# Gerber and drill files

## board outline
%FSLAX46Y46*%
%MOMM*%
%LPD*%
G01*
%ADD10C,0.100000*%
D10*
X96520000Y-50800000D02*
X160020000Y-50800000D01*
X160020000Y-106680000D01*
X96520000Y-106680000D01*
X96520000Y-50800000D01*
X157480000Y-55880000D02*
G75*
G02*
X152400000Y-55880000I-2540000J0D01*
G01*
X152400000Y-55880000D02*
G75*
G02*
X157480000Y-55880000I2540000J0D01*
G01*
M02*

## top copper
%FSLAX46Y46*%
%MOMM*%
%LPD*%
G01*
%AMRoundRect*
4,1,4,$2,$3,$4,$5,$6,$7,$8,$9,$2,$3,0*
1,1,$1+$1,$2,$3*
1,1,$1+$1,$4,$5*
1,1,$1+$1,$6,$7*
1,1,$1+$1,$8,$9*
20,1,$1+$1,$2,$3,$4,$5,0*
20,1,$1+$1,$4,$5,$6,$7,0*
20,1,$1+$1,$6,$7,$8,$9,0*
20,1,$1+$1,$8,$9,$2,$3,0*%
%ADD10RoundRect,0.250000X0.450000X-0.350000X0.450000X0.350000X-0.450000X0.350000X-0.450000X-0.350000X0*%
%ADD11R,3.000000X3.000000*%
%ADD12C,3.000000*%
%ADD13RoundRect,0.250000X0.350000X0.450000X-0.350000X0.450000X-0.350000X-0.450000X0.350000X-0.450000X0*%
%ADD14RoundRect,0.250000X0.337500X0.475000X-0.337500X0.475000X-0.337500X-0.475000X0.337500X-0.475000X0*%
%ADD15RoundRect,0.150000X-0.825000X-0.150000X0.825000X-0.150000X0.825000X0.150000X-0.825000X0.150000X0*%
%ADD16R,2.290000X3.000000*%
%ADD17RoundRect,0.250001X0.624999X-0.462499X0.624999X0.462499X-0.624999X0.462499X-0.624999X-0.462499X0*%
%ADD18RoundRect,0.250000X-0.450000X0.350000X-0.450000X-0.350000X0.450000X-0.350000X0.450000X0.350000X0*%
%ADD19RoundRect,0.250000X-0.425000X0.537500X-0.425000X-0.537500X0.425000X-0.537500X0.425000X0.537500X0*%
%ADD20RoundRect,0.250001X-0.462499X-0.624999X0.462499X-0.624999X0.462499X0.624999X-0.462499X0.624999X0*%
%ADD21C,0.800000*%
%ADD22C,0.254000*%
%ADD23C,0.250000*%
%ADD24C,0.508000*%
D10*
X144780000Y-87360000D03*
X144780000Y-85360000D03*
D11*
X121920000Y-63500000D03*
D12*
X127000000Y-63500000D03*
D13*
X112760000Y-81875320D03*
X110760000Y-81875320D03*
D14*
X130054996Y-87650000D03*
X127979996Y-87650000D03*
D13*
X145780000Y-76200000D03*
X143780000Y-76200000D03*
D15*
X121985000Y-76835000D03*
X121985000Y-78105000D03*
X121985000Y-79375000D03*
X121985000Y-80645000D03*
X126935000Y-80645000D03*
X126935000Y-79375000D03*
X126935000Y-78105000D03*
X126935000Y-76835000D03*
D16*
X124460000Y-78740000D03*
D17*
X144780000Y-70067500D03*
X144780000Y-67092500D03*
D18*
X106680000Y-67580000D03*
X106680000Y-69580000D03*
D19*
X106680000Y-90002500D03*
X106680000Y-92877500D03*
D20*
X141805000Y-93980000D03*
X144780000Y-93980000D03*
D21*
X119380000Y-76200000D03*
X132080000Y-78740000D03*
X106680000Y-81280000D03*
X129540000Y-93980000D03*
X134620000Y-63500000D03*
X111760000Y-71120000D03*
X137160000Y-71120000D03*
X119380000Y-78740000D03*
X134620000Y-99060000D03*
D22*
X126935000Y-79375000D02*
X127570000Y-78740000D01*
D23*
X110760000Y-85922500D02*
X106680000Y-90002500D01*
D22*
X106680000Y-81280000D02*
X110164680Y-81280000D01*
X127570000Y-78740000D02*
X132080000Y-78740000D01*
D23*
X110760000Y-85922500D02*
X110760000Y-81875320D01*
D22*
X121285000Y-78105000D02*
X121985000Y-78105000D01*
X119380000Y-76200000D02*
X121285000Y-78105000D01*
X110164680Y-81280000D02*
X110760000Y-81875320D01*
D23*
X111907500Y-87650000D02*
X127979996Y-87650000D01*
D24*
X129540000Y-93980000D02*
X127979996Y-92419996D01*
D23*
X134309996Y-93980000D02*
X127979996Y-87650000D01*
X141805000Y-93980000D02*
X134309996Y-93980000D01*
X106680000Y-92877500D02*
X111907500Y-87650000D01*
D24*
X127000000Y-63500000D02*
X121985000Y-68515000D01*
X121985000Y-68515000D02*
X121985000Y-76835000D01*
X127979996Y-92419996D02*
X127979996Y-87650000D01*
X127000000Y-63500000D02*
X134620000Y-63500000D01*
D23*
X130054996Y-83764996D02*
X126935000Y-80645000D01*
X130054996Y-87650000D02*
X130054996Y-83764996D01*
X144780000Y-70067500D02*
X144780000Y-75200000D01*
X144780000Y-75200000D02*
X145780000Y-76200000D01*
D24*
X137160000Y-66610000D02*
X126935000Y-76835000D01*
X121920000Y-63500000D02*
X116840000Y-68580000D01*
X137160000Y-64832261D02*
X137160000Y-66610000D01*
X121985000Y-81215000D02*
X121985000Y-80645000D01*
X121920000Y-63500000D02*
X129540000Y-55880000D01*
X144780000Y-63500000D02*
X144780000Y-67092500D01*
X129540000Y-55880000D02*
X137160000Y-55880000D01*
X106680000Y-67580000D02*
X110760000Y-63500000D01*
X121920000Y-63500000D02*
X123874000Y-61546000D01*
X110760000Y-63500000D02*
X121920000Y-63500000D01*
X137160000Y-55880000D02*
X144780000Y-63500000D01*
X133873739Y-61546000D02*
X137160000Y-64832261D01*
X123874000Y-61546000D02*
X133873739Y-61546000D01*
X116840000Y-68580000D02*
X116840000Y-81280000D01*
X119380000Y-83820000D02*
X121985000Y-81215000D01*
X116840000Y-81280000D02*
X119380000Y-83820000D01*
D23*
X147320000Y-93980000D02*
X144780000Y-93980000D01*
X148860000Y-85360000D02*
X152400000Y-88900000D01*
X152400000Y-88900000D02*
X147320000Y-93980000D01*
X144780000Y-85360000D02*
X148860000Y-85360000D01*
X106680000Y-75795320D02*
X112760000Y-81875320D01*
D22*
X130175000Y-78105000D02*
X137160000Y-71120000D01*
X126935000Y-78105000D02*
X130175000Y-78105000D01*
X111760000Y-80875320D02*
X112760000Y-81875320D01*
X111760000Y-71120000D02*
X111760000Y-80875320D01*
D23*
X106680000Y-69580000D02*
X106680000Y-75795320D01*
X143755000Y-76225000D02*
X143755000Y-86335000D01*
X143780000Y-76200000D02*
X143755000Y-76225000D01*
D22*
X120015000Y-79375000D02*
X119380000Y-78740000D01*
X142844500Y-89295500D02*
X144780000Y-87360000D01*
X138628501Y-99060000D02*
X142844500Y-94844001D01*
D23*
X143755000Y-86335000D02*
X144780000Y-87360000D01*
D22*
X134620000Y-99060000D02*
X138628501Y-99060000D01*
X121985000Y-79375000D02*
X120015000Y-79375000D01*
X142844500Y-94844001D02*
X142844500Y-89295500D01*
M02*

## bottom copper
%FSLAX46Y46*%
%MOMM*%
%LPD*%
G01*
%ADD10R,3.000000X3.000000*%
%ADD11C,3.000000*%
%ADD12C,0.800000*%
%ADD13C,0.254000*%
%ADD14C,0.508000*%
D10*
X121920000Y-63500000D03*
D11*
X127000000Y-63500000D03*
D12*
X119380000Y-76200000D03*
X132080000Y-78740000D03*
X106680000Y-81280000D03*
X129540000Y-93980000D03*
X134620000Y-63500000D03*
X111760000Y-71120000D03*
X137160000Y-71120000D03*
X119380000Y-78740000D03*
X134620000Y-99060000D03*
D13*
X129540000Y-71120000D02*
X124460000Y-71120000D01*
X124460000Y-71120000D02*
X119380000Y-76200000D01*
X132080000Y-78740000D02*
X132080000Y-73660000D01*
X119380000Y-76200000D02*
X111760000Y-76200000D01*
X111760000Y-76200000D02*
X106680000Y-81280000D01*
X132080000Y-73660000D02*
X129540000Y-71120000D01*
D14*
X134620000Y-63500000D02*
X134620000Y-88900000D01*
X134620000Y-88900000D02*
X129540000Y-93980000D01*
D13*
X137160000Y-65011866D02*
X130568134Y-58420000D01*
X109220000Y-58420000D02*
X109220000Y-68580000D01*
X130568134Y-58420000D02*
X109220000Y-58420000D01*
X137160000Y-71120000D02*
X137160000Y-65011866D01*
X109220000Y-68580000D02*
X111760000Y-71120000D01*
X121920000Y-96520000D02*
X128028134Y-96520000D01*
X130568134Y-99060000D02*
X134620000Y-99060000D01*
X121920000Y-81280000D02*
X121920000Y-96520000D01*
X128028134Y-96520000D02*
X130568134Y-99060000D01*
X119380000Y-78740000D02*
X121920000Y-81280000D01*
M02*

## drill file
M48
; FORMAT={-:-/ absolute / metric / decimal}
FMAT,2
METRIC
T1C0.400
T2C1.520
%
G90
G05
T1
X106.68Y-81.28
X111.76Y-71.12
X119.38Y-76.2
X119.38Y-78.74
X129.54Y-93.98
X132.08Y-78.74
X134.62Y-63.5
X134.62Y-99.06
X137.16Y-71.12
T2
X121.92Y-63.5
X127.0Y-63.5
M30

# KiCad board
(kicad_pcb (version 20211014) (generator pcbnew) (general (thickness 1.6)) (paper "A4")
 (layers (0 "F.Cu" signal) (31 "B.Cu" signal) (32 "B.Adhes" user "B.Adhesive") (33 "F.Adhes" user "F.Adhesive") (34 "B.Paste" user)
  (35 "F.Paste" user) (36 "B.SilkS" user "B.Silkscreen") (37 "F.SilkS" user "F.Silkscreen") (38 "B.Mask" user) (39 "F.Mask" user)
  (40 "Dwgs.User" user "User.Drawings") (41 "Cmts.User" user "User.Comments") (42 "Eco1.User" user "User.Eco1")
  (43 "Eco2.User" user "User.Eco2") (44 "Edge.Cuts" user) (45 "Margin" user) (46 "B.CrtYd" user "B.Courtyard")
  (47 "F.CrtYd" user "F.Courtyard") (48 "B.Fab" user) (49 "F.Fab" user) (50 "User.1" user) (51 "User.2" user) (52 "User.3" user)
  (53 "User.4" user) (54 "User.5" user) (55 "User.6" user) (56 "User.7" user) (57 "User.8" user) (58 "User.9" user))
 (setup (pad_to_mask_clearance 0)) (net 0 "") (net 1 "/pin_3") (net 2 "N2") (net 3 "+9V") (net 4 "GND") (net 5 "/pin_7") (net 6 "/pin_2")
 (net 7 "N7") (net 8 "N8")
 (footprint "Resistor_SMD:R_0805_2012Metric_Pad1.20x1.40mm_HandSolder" (layer "F.Cu") (at 144.78 86.36 90)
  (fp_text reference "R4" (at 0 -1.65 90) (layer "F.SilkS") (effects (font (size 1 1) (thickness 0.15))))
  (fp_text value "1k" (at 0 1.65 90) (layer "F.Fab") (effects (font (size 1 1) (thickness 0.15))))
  (pad "1" smd roundrect (at -1 0 90) (size 1.2 1.4) (layers "F.Cu" "F.Paste" "F.Mask") (roundrect_rratio 0.208333) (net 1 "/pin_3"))
  (pad "2" smd roundrect (at 1 0 90) (size 1.2 1.4) (layers "F.Cu" "F.Paste" "F.Mask") (roundrect_rratio 0.208333) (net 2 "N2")))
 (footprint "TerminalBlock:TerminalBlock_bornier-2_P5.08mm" (layer "F.Cu") (at 121.92 63.5)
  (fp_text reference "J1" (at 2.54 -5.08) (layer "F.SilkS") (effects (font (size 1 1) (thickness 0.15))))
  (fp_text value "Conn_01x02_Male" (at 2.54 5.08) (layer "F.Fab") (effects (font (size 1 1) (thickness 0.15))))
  (pad "1" thru_hole rect (at 0 0) (size 3 3) (drill 1.52) (layers *.Cu *.Mask) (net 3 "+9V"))
  (pad "2" thru_hole circle (at 5.08 0) (size 3 3) (drill 1.52) (layers *.Cu *.Mask) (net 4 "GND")))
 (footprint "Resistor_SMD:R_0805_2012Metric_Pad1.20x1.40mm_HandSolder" (layer "F.Cu") (at 111.76 81.87532 180)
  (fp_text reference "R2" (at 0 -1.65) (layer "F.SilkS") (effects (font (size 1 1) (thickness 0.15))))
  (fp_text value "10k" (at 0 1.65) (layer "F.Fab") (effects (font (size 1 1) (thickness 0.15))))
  (pad "1" smd roundrect (at -1 0 180) (size 1.2 1.4) (layers "F.Cu" "F.Paste" "F.Mask") (roundrect_rratio 0.208333) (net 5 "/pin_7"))
  (pad "2" smd roundrect (at 1 0 180) (size 1.2 1.4) (layers "F.Cu" "F.Paste" "F.Mask") (roundrect_rratio 0.208333) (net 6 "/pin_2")))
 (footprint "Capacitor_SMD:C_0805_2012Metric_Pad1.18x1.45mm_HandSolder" (layer "F.Cu") (at 129.017496 87.65 180)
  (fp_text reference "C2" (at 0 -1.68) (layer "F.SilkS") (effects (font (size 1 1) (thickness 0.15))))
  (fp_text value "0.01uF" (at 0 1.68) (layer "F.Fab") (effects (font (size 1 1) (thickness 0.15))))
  (pad "1" smd roundrect (at -1.0375 0 180) (size 1.175 1.45) (layers "F.Cu" "F.Paste" "F.Mask") (roundrect_rratio 0.212766) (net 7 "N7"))
  (pad "2" smd roundrect (at 1.0375 0 180) (size 1.175 1.45) (layers "F.Cu" "F.Paste" "F.Mask") (roundrect_rratio 0.212766) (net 4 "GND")))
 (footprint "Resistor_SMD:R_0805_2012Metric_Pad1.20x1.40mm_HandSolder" (layer "F.Cu") (at 144.78 76.2 180)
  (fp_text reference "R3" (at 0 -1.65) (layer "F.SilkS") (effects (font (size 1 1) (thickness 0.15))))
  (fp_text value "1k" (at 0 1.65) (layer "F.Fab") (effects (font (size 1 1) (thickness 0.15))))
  (pad "1" smd roundrect (at -1 0 180) (size 1.2 1.4) (layers "F.Cu" "F.Paste" "F.Mask") (roundrect_rratio 0.208333) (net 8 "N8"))
  (pad "2" smd roundrect (at 1 0 180) (size 1.2 1.4) (layers "F.Cu" "F.Paste" "F.Mask") (roundrect_rratio 0.208333) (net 1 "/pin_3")))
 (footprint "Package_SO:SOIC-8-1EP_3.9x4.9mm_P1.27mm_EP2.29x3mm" (layer "F.Cu") (at 124.46 78.74)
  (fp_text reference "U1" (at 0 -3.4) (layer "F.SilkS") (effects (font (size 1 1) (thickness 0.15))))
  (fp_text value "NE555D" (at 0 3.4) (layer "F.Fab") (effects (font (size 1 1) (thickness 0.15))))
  (pad "" smd roundrect (at 0.57 -0.75) (size 0.92 1.21) (layers "F.Paste") (roundrect_rratio 0.25))
  (pad "" smd roundrect (at -0.57 0.75) (size 0.92 1.21) (layers "F.Paste") (roundrect_rratio 0.25))
  (pad "" smd roundrect (at 0.57 0.75) (size 0.92 1.21) (layers "F.Paste") (roundrect_rratio 0.25))
  (pad "" smd roundrect (at -0.57 -0.75) (size 0.92 1.21) (layers "F.Paste") (roundrect_rratio 0.25))
  (pad "1" smd roundrect (at -2.475 -1.905) (size 1.95 0.6) (layers "F.Cu" "F.Paste" "F.Mask") (roundrect_rratio 0.25) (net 4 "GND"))
  (pad "2" smd roundrect (at -2.475 -0.635) (size 1.95 0.6) (layers "F.Cu" "F.Paste" "F.Mask") (roundrect_rratio 0.25) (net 6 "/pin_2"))
  (pad "3" smd roundrect (at -2.475 0.635) (size 1.95 0.6) (layers "F.Cu" "F.Paste" "F.Mask") (roundrect_rratio 0.25) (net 1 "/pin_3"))
  (pad "4" smd roundrect (at -2.475 1.905) (size 1.95 0.6) (layers "F.Cu" "F.Paste" "F.Mask") (roundrect_rratio 0.25) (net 3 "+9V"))
  (pad "5" smd roundrect (at 2.475 1.905) (size 1.95 0.6) (layers "F.Cu" "F.Paste" "F.Mask") (roundrect_rratio 0.25) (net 7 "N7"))
  (pad "6" smd roundrect (at 2.475 0.635) (size 1.95 0.6) (layers "F.Cu" "F.Paste" "F.Mask") (roundrect_rratio 0.25) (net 6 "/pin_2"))
  (pad "7" smd roundrect (at 2.475 -0.635) (size 1.95 0.6) (layers "F.Cu" "F.Paste" "F.Mask") (roundrect_rratio 0.25) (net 5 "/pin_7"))
  (pad "8" smd roundrect (at 2.475 -1.905) (size 1.95 0.6) (layers "F.Cu" "F.Paste" "F.Mask") (roundrect_rratio 0.25) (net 3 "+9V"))
  (pad "9" smd rect (at 0 0) (size 2.29 3) (layers "F.Cu" "F.Mask")))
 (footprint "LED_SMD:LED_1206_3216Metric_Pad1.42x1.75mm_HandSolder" (layer "F.Cu") (at 144.78 68.58 90)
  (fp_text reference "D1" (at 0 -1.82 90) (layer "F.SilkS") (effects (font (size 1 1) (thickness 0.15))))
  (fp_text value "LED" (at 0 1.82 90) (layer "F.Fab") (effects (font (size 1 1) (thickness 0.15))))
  (pad "1" smd roundrect (at -1.4875 0 90) (size 1.425 1.75) (layers "F.Cu" "F.Paste" "F.Mask") (roundrect_rratio 0.175439) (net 8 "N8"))
  (pad "2" smd roundrect (at 1.4875 0 90) (size 1.425 1.75) (layers "F.Cu" "F.Paste" "F.Mask") (roundrect_rratio 0.175439) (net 3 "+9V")))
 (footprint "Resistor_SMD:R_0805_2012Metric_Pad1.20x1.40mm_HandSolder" (layer "F.Cu") (at 106.68 68.58 -90)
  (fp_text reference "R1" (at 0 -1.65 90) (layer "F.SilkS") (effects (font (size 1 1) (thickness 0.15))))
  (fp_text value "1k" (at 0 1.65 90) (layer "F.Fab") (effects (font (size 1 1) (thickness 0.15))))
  (pad "1" smd roundrect (at -1 0 270) (size 1.2 1.4) (layers "F.Cu" "F.Paste" "F.Mask") (roundrect_rratio 0.208333) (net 3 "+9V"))
  (pad "2" smd roundrect (at 1 0 270) (size 1.2 1.4) (layers "F.Cu" "F.Paste" "F.Mask") (roundrect_rratio 0.208333) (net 5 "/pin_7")))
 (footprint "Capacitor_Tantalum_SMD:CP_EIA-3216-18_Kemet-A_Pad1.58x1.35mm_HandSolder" (layer "F.Cu") (at 106.68 91.44 -90)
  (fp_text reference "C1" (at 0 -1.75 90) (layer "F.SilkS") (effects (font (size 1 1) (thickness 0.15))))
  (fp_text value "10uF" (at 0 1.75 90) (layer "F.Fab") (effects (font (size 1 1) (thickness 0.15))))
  (pad "1" smd roundrect (at -1.4375 0 270) (size 1.575 1.35) (layers "F.Cu" "F.Paste" "F.Mask") (roundrect_rratio 0.185185)
   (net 6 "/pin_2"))
  (pad "2" smd roundrect (at 1.4375 0 270) (size 1.575 1.35) (layers "F.Cu" "F.Paste" "F.Mask") (roundrect_rratio 0.185185) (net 4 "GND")))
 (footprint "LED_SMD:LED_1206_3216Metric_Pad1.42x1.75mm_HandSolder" (layer "F.Cu") (at 143.2925 93.98)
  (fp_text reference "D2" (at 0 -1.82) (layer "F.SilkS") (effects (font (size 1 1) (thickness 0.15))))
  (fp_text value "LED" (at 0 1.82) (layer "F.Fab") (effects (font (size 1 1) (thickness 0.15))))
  (pad "1" smd roundrect (at -1.4875 0) (size 1.425 1.75) (layers "F.Cu" "F.Paste" "F.Mask") (roundrect_rratio 0.175439) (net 4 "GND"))
  (pad "2" smd roundrect (at 1.4875 0) (size 1.425 1.75) (layers "F.Cu" "F.Paste" "F.Mask") (roundrect_rratio 0.175439) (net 2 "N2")))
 (gr_rect (start 96.52 50.8) (end 160.02 106.68) (layer "Edge.Cuts") (width 0.1) (fill none))
 (gr_circle (center 154.94 55.88) (end 154.94 53.34) (layer "Edge.Cuts") (width 0.1) (fill none))
 (segment (start 126.935 79.375) (end 127.57 78.74) (width 0.254) (layer "F.Cu") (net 6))
 (segment (start 110.76 85.9225) (end 106.68 90.0025) (width 0.25) (layer "F.Cu") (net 6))
 (segment (start 106.68 81.28) (end 110.16468 81.28) (width 0.254) (layer "F.Cu") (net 6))
 (segment (start 127.57 78.74) (end 132.08 78.74) (width 0.254) (layer "F.Cu") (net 6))
 (segment (start 110.76 85.9225) (end 110.76 81.87532) (width 0.25) (layer "F.Cu") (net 6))
 (segment (start 121.285 78.105) (end 121.985 78.105) (width 0.254) (layer "F.Cu") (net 6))
 (segment (start 119.38 76.2) (end 121.285 78.105) (width 0.254) (layer "F.Cu") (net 6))
 (segment (start 110.16468 81.28) (end 110.76 81.87532) (width 0.254) (layer "F.Cu") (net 6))
 (via (at 119.38 76.2) (size 0.8) (drill 0.4) (layers "F.Cu" "B.Cu") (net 6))
 (via (at 132.08 78.74) (size 0.8) (drill 0.4) (layers "F.Cu" "B.Cu") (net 6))
 (via (at 106.68 81.28) (size 0.8) (drill 0.4) (layers "F.Cu" "B.Cu") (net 6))
 (segment (start 129.54 71.12) (end 124.46 71.12) (width 0.254) (layer "B.Cu") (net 6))
 (segment (start 124.46 71.12) (end 119.38 76.2) (width 0.254) (layer "B.Cu") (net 6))
 (segment (start 132.08 78.74) (end 132.08 73.66) (width 0.254) (layer "B.Cu") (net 6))
 (segment (start 119.38 76.2) (end 111.76 76.2) (width 0.254) (layer "B.Cu") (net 6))
 (segment (start 111.76 76.2) (end 106.68 81.28) (width 0.254) (layer "B.Cu") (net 6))
 (segment (start 132.08 73.66) (end 129.54 71.12) (width 0.254) (layer "B.Cu") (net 6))
 (segment (start 111.9075 87.65) (end 127.979996 87.65) (width 0.25) (layer "F.Cu") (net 4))
 (segment (start 129.54 93.98) (end 127.979996 92.419996) (width 0.508) (layer "F.Cu") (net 4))
 (segment (start 134.309996 93.98) (end 127.979996 87.65) (width 0.25) (layer "F.Cu") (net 4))
 (segment (start 141.805 93.98) (end 134.309996 93.98) (width 0.25) (layer "F.Cu") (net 4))
 (segment (start 106.68 92.8775) (end 111.9075 87.65) (width 0.25) (layer "F.Cu") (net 4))
 (segment (start 127 63.5) (end 121.985 68.515) (width 0.508) (layer "F.Cu") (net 4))
 (segment (start 121.985 68.515) (end 121.985 76.835) (width 0.508) (layer "F.Cu") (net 4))
 (segment (start 127.979996 92.419996) (end 127.979996 87.65) (width 0.508) (layer "F.Cu") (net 4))
 (segment (start 127 63.5) (end 134.62 63.5) (width 0.508) (layer "F.Cu") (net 4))
 (via (at 129.54 93.98) (size 0.8) (drill 0.4) (layers "F.Cu" "B.Cu") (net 4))
 (via (at 134.62 63.5) (size 0.8) (drill 0.4) (layers "F.Cu" "B.Cu") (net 4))
 (segment (start 134.62 63.5) (end 134.62 88.9) (width 0.508) (layer "B.Cu") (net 4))
 (segment (start 134.62 88.9) (end 129.54 93.98) (width 0.508) (layer "B.Cu") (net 4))
 (segment (start 130.054996 83.764996) (end 126.935 80.645) (width 0.25) (layer "F.Cu") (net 7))
 (segment (start 130.054996 87.65) (end 130.054996 83.764996) (width 0.25) (layer "F.Cu") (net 7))
 (segment (start 144.78 70.0675) (end 144.78 75.2) (width 0.25) (layer "F.Cu") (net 8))
 (segment (start 144.78 75.2) (end 145.78 76.2) (width 0.25) (layer "F.Cu") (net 8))
 (segment (start 137.16 66.61) (end 126.935 76.835) (width 0.508) (layer "F.Cu") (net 3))
 (segment (start 121.92 63.5) (end 116.84 68.58) (width 0.508) (layer "F.Cu") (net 3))
 (segment (start 137.16 64.832261) (end 137.16 66.61) (width 0.508) (layer "F.Cu") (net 3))
 (segment (start 121.985 81.215) (end 121.985 80.645) (width 0.508) (layer "F.Cu") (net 3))
 (segment (start 121.92 63.5) (end 129.54 55.88) (width 0.508) (layer "F.Cu") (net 3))
 (segment (start 144.78 63.5) (end 144.78 67.0925) (width 0.508) (layer "F.Cu") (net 3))
 (segment (start 129.54 55.88) (end 137.16 55.88) (width 0.508) (layer "F.Cu") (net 3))
 (segment (start 106.68 67.58) (end 110.76 63.5) (width 0.508) (layer "F.Cu") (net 3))
 (segment (start 121.92 63.5) (end 123.874 61.546) (width 0.508) (layer "F.Cu") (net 3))
 (segment (start 110.76 63.5) (end 121.92 63.5) (width 0.508) (layer "F.Cu") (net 3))
 (segment (start 137.16 55.88) (end 144.78 63.5) (width 0.508) (layer "F.Cu") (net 3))
 (segment (start 133.873739 61.546) (end 137.16 64.832261) (width 0.508) (layer "F.Cu") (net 3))
 (segment (start 123.874 61.546) (end 133.873739 61.546) (width 0.508) (layer "F.Cu") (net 3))
 (segment (start 116.84 68.58) (end 116.84 81.28) (width 0.508) (layer "F.Cu") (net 3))
 (segment (start 119.38 83.82) (end 121.985 81.215) (width 0.508) (layer "F.Cu") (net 3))
 (segment (start 116.84 81.28) (end 119.38 83.82) (width 0.508) (layer "F.Cu") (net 3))
 (segment (start 147.32 93.98) (end 144.78 93.98) (width 0.25) (layer "F.Cu") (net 2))
 (segment (start 148.86 85.36) (end 152.4 88.9) (width 0.25) (layer "F.Cu") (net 2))
 (segment (start 152.4 88.9) (end 147.32 93.98) (width 0.25) (layer "F.Cu") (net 2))
 (segment (start 144.78 85.36) (end 148.86 85.36) (width 0.25) (layer "F.Cu") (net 2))
 (segment (start 106.68 75.79532) (end 112.76 81.87532) (width 0.25) (layer "F.Cu") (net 5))
 (segment (start 130.175 78.105) (end 137.16 71.12) (width 0.254) (layer "F.Cu") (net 5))
 (segment (start 126.935 78.105) (end 130.175 78.105) (width 0.254) (layer "F.Cu") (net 5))
 (segment (start 111.76 80.87532) (end 112.76 81.87532) (width 0.254) (layer "F.Cu") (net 5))
 (segment (start 111.76 71.12) (end 111.76 80.87532) (width 0.254) (layer "F.Cu") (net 5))
 (segment (start 106.68 69.58) (end 106.68 75.79532) (width 0.25) (layer "F.Cu") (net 5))
 (via (at 111.76 71.12) (size 0.8) (drill 0.4) (layers "F.Cu" "B.Cu") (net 5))
 (via (at 137.16 71.12) (size 0.8) (drill 0.4) (layers "F.Cu" "B.Cu") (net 5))
 (segment (start 137.16 65.011866) (end 130.568134 58.42) (width 0.254) (layer "B.Cu") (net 5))
 (segment (start 109.22 58.42) (end 109.22 68.58) (width 0.254) (layer "B.Cu") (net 5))
 (segment (start 130.568134 58.42) (end 109.22 58.42) (width 0.254) (layer "B.Cu") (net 5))
 (segment (start 137.16 71.12) (end 137.16 65.011866) (width 0.254) (layer "B.Cu") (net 5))
 (segment (start 109.22 68.58) (end 111.76 71.12) (width 0.254) (layer "B.Cu") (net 5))
 (segment (start 143.755 76.225) (end 143.755 86.335) (width 0.25) (layer "F.Cu") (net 1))
 (segment (start 143.78 76.2) (end 143.755 76.225) (width 0.25) (layer "F.Cu") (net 1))
 (segment (start 120.015 79.375) (end 119.38 78.74) (width 0.254) (layer "F.Cu") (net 1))
 (segment (start 142.8445 89.2955) (end 144.78 87.36) (width 0.254) (layer "F.Cu") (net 1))
 (segment (start 138.628501 99.06) (end 142.8445 94.844001) (width 0.254) (layer "F.Cu") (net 1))
 (segment (start 143.755 86.335) (end 144.78 87.36) (width 0.25) (layer "F.Cu") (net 1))
 (segment (start 134.62 99.06) (end 138.628501 99.06) (width 0.254) (layer "F.Cu") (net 1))
 (segment (start 121.985 79.375) (end 120.015 79.375) (width 0.254) (layer "F.Cu") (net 1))
 (segment (start 142.8445 94.844001) (end 142.8445 89.2955) (width 0.254) (layer "F.Cu") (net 1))
 (via (at 119.38 78.74) (size 0.8) (drill 0.4) (layers "F.Cu" "B.Cu") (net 1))
 (via (at 134.62 99.06) (size 0.8) (drill 0.4) (layers "F.Cu" "B.Cu") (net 1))
 (segment (start 121.92 96.52) (end 128.028134 96.52) (width 0.254) (layer "B.Cu") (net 1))
 (segment (start 130.568134 99.06) (end 134.62 99.06) (width 0.254) (layer "B.Cu") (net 1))
 (segment (start 121.92 81.28) (end 121.92 96.52) (width 0.254) (layer "B.Cu") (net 1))
 (segment (start 128.028134 96.52) (end 130.568134 99.06) (width 0.254) (layer "B.Cu") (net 1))
 (segment (start 119.38 78.74) (end 121.92 81.28) (width 0.254) (layer "B.Cu") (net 1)))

